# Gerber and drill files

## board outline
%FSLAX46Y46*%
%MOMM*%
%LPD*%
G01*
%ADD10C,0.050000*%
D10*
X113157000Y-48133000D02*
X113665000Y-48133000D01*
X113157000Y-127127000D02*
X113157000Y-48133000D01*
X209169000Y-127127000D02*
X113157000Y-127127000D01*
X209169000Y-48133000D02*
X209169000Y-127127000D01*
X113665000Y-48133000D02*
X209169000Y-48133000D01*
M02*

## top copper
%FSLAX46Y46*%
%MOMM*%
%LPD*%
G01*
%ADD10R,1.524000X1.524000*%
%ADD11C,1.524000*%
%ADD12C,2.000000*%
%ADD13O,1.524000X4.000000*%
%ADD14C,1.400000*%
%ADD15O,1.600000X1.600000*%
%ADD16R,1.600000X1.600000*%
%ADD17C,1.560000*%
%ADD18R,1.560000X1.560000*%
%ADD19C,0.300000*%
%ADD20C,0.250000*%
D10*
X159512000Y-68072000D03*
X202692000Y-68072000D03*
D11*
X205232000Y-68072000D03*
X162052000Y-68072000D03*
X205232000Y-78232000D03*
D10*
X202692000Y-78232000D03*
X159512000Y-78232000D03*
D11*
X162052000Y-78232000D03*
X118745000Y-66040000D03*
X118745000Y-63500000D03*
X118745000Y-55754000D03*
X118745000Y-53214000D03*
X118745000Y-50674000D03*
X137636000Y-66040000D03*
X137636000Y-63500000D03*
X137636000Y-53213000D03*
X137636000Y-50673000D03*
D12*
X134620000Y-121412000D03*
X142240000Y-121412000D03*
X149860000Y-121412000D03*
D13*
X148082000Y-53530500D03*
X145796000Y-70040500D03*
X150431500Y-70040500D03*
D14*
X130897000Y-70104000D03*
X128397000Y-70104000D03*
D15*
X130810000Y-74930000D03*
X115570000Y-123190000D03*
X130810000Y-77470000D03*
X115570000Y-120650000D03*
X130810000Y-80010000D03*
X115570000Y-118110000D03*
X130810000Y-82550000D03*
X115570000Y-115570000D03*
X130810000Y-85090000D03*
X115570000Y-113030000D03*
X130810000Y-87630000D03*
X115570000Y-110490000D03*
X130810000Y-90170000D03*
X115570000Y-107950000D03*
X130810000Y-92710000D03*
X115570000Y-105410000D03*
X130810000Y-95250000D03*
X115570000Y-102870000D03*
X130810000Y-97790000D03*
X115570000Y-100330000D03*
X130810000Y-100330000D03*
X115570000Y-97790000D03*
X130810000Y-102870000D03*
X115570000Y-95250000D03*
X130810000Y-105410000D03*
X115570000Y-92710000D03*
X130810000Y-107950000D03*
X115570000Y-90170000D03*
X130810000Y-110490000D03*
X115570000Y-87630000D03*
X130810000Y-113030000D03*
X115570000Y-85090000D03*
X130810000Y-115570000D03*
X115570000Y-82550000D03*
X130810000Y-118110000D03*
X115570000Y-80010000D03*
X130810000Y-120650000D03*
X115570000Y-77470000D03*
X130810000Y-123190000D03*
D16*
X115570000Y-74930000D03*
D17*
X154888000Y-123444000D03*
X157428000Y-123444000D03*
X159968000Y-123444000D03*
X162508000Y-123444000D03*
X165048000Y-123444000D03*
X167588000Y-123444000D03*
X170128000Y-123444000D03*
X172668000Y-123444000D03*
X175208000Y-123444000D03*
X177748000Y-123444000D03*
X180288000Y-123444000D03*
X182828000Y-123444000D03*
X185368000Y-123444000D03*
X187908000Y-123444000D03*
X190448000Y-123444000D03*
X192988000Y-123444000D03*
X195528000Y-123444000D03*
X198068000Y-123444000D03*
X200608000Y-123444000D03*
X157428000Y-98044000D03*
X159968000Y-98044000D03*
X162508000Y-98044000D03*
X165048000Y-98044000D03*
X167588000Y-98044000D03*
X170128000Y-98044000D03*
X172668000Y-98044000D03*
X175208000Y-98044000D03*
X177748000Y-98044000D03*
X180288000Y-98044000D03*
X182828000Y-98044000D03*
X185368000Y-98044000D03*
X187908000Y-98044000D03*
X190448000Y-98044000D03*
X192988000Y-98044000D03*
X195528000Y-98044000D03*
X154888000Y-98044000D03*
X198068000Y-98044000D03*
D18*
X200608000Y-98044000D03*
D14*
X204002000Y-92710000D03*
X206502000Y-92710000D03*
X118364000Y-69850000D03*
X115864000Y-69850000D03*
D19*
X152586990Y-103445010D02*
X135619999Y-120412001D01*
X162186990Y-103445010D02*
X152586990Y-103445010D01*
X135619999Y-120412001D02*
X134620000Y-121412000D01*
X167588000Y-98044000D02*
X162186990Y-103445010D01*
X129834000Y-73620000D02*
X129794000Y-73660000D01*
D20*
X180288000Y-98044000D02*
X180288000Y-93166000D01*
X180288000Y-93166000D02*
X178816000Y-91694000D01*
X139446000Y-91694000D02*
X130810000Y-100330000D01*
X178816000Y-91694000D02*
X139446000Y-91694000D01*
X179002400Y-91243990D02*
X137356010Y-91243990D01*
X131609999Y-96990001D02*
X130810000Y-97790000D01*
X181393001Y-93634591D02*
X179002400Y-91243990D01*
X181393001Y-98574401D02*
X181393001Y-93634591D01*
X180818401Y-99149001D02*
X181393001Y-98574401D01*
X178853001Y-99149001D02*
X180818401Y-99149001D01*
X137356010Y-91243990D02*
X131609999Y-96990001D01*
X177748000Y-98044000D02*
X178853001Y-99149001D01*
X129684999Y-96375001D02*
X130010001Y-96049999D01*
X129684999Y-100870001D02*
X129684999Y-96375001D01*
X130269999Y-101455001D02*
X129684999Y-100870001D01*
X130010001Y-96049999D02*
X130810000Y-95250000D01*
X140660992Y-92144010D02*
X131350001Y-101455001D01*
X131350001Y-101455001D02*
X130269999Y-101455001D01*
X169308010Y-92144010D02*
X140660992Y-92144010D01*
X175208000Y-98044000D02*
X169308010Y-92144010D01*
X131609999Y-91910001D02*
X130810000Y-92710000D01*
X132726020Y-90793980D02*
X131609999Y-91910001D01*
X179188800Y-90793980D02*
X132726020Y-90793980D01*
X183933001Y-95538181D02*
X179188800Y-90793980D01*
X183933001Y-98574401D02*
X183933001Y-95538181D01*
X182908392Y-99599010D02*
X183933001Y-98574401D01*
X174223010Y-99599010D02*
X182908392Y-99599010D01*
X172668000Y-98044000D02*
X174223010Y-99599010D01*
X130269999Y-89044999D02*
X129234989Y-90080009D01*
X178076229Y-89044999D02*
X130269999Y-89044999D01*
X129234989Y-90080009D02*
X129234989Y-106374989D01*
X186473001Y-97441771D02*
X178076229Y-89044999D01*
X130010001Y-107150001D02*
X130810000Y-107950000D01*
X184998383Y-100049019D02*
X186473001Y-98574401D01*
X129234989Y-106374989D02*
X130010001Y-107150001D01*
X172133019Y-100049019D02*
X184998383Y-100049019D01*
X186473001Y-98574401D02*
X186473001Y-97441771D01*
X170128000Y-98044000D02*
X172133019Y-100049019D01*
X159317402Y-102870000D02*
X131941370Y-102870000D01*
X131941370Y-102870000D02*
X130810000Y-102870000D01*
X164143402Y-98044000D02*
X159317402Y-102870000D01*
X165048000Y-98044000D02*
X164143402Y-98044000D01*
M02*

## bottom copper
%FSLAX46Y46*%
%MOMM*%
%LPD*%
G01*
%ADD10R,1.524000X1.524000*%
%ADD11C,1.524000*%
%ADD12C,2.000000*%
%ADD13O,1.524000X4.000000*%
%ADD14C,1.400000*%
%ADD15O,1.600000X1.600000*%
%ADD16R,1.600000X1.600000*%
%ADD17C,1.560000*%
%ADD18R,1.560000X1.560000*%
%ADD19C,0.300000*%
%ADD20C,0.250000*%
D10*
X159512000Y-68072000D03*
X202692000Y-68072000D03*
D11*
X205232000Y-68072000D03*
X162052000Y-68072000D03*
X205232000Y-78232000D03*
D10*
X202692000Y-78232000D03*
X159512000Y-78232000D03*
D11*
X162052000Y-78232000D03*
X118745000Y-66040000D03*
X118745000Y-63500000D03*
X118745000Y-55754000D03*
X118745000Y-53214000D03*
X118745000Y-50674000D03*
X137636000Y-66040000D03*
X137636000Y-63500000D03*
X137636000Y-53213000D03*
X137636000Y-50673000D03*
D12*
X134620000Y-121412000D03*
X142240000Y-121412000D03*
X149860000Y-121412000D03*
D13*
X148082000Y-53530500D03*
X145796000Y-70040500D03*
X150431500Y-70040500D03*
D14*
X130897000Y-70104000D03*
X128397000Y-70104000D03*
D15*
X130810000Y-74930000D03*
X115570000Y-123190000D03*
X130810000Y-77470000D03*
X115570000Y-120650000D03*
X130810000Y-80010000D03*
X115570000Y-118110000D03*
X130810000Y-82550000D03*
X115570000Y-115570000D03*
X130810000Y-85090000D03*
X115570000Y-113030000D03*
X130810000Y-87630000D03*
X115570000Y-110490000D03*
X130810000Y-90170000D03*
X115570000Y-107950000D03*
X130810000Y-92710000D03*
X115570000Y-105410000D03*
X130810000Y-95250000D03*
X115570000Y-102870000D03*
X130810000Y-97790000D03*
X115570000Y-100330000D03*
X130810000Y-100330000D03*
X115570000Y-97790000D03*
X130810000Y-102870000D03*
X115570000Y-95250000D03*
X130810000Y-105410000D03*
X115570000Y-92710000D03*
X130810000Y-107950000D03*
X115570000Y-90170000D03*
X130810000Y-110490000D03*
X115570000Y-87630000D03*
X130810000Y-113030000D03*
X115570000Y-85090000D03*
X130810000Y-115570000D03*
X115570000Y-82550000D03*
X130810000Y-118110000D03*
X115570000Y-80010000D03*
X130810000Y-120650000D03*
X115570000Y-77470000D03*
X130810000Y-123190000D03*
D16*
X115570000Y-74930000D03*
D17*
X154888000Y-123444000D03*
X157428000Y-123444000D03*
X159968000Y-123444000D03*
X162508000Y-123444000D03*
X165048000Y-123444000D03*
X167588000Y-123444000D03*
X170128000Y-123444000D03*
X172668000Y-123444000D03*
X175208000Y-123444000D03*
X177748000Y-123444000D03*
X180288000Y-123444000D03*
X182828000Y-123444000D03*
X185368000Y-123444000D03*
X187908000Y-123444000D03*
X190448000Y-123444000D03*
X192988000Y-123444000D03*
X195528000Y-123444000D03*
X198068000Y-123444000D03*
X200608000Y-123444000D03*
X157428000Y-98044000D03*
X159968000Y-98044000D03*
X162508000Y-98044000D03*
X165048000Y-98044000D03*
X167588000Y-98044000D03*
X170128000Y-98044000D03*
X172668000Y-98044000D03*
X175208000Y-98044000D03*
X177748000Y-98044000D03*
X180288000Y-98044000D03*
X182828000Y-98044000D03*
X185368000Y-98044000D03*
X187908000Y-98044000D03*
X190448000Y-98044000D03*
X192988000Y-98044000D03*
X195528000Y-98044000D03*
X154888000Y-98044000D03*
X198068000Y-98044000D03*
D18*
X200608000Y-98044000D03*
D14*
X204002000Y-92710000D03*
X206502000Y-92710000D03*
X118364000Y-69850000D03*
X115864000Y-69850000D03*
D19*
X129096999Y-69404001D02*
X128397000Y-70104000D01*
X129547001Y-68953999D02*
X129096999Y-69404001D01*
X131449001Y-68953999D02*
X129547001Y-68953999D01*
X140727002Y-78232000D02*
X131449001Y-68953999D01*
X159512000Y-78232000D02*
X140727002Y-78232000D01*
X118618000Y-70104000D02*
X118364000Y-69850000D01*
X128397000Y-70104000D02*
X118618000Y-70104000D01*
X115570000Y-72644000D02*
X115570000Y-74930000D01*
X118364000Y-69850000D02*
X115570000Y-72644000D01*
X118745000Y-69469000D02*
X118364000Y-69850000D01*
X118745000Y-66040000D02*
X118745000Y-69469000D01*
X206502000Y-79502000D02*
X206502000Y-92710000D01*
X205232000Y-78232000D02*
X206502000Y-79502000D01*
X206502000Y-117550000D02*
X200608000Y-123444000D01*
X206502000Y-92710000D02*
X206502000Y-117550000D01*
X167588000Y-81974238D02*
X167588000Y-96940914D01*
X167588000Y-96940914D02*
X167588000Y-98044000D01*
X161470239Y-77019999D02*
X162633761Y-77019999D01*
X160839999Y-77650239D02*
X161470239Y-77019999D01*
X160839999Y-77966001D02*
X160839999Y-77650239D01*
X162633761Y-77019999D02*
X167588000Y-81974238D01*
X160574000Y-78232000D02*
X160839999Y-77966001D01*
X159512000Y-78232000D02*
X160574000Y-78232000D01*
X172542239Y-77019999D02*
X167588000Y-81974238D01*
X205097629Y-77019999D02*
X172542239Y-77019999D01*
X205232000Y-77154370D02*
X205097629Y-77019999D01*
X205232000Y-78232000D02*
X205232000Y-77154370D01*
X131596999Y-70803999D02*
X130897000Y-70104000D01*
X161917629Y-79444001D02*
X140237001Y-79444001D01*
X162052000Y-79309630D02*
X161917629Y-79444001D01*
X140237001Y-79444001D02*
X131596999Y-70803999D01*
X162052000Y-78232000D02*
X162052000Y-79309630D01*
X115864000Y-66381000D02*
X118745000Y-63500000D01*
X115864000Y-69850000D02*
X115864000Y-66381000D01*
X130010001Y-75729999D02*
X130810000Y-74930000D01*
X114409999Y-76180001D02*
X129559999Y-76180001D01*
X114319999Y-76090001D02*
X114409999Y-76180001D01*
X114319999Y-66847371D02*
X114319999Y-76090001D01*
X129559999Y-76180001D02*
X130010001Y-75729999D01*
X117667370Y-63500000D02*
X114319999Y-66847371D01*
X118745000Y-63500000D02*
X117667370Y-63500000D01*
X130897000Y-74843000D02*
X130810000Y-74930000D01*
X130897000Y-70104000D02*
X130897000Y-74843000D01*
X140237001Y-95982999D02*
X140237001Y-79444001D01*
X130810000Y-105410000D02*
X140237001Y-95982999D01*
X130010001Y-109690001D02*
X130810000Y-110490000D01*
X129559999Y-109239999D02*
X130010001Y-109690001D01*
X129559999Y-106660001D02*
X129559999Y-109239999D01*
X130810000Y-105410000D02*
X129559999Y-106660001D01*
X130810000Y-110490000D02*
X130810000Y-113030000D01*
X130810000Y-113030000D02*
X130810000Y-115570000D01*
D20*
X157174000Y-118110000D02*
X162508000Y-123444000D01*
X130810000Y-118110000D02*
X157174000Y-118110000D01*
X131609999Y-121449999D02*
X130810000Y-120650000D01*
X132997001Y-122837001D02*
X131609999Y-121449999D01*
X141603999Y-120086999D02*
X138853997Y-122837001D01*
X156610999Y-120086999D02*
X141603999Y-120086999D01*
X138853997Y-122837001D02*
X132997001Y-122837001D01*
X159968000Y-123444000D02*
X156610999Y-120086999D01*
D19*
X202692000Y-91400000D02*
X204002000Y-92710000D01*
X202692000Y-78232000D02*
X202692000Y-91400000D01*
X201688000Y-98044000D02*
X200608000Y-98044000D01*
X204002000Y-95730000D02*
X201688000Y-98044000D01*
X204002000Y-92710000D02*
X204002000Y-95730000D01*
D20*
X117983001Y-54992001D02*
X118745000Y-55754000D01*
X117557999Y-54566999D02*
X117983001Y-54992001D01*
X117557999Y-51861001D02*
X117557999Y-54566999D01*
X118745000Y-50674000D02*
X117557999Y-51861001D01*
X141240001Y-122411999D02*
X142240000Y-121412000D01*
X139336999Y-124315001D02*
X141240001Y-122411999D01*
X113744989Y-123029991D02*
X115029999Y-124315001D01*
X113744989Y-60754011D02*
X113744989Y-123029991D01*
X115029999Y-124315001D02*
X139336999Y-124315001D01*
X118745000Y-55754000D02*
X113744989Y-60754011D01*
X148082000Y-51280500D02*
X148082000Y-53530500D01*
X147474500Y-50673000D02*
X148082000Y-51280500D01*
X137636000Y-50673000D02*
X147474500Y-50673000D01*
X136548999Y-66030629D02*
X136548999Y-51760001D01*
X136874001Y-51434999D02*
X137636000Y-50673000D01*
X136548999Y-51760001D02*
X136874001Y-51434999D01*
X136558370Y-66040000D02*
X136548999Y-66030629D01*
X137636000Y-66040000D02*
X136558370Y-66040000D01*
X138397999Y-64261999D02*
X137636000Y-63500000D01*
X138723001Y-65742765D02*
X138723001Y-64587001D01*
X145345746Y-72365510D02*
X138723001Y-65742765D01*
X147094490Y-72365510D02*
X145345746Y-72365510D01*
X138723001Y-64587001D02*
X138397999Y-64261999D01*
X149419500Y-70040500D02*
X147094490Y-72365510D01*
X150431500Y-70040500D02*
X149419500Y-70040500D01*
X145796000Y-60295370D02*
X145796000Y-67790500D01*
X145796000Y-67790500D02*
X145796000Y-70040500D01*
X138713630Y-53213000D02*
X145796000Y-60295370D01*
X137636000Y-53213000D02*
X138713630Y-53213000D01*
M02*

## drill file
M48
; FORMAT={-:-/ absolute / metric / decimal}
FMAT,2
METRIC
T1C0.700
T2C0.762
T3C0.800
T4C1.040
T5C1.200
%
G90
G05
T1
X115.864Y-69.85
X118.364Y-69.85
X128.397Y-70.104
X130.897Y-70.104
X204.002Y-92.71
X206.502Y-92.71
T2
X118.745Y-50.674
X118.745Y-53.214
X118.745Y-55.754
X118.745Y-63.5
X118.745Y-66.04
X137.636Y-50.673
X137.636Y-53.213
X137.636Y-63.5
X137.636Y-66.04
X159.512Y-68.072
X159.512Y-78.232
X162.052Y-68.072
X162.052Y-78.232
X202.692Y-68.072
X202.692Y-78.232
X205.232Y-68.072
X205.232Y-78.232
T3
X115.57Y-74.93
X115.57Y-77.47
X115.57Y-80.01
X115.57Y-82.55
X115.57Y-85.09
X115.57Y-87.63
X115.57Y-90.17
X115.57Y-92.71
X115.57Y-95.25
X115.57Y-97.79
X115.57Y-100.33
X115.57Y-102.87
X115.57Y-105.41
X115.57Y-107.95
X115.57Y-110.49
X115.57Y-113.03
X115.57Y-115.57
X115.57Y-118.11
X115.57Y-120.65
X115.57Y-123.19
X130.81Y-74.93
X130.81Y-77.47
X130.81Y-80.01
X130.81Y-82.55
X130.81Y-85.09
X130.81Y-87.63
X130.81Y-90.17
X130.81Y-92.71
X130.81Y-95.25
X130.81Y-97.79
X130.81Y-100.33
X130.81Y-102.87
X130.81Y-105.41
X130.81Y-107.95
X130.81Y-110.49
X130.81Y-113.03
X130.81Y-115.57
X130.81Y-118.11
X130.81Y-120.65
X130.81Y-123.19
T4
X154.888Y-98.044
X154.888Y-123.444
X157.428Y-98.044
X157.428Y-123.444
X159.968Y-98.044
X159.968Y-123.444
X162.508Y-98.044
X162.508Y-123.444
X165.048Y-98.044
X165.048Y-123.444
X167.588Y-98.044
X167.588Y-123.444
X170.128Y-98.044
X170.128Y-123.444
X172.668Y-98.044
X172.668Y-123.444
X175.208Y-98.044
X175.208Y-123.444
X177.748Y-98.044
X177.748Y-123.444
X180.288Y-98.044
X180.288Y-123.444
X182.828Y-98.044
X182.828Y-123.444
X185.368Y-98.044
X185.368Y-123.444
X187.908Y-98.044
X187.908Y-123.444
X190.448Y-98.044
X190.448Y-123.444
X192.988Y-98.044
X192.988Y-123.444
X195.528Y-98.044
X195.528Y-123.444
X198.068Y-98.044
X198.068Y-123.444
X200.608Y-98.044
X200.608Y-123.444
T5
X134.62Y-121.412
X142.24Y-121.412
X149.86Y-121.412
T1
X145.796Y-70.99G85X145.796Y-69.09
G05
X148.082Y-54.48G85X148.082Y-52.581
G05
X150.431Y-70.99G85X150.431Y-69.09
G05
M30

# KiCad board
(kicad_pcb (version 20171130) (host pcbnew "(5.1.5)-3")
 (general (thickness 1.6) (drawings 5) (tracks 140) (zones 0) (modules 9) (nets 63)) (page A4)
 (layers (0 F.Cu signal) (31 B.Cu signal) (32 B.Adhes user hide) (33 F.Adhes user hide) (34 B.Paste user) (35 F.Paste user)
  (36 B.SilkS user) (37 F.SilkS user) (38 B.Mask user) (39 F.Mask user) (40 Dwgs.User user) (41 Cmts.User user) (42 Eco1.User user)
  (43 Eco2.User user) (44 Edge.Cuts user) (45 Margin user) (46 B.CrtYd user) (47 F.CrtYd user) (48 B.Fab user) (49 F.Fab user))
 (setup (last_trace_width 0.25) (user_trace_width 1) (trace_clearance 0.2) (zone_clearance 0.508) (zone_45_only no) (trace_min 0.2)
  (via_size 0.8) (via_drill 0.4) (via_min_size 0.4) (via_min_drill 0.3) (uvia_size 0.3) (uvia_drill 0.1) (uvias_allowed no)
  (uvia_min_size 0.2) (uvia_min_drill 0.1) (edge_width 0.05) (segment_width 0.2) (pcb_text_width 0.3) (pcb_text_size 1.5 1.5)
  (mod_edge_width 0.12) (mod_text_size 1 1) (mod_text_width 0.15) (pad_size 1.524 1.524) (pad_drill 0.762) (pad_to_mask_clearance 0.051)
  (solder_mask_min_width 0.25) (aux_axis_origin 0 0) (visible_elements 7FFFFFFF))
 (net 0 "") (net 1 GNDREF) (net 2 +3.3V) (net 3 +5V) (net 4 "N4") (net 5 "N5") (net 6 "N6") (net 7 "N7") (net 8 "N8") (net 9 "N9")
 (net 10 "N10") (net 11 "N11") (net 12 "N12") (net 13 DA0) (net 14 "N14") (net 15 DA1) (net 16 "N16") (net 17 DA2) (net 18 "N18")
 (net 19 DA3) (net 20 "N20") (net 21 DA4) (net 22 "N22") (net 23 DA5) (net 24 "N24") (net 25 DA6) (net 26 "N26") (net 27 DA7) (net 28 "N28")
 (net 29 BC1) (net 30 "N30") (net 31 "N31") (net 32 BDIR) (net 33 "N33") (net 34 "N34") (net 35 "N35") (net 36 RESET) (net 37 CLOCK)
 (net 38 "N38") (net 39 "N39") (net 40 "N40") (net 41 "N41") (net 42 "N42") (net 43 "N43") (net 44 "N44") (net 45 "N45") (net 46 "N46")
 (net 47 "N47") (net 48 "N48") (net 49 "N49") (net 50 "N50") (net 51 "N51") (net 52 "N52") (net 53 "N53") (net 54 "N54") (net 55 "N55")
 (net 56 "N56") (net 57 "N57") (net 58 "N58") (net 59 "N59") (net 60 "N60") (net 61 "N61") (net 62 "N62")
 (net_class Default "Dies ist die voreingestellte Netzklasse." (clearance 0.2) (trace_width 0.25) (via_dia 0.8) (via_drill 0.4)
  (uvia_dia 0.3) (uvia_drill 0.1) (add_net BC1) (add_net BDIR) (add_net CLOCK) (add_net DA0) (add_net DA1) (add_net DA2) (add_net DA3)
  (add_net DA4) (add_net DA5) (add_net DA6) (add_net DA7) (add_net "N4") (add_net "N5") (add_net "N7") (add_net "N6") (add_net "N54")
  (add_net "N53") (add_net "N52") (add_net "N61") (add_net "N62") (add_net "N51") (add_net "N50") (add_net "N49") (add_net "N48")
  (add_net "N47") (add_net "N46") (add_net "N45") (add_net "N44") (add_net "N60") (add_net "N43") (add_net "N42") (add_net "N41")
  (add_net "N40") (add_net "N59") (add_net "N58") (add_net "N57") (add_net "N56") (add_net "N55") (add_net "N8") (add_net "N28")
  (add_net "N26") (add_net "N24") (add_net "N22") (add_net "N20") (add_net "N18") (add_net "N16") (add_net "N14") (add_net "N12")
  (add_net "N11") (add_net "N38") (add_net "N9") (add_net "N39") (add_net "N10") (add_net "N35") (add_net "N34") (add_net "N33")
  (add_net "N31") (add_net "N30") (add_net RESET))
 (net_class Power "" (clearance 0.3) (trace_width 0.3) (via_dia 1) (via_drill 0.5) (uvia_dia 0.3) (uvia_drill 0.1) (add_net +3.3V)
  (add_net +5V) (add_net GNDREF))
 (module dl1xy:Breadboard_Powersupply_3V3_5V (layer F.Cu) (at 182.372 60.198)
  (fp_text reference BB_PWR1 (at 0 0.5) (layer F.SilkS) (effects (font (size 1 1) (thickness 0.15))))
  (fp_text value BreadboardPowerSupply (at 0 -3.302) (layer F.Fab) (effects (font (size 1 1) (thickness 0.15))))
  (pad 5 thru_hole rect (at -22.86 7.874) (size 1.524 1.524) (drill 0.762) (layers *.Cu *.Mask))
  (pad 7 thru_hole rect (at 20.32 7.874) (size 1.524 1.524) (drill 0.762) (layers *.Cu *.Mask))
  (pad 8 thru_hole circle (at 22.86 7.874) (size 1.524 1.524) (drill 0.762) (layers *.Cu *.Mask))
  (pad 6 thru_hole circle (at -20.32 7.874) (size 1.524 1.524) (drill 0.762) (layers *.Cu *.Mask))
  (pad 4 thru_hole circle (at 22.86 18.034) (size 1.524 1.524) (drill 0.762) (layers *.Cu *.Mask) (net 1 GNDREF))
  (pad 3 thru_hole rect (at 20.32 18.034) (size 1.524 1.524) (drill 0.762) (layers *.Cu *.Mask) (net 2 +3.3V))
  (pad 2 thru_hole rect (at -22.86 18.034) (size 1.524 1.524) (drill 0.762) (layers *.Cu *.Mask) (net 1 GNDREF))
  (pad 1 thru_hole circle (at -20.32 18.034) (size 1.524 1.524) (drill 0.762) (layers *.Cu *.Mask) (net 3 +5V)))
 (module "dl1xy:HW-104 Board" (layer F.Cu) (at 140.716 58.42 270)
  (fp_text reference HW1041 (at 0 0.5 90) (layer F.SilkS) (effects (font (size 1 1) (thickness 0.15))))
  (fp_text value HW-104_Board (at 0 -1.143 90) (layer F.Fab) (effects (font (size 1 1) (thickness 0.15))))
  (pad 5 thru_hole circle (at 7.62 21.971 270) (size 1.524 1.524) (drill 0.762) (layers *.Cu *.Mask) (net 1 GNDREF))
  (pad 4 thru_hole circle (at 5.08 21.971 270) (size 1.524 1.524) (drill 0.762) (layers *.Cu *.Mask) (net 3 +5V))
  (pad 3 thru_hole circle (at -2.666 21.971 270) (size 1.524 1.524) (drill 0.762) (layers *.Cu *.Mask) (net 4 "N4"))
  (pad 2 thru_hole circle (at -5.206 21.971 270) (size 1.524 1.524) (drill 0.762) (layers *.Cu *.Mask) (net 1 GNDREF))
  (pad 1 thru_hole circle (at -7.746 21.971 270) (size 1.524 1.524) (drill 0.762) (layers *.Cu *.Mask) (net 4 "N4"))
  (pad 9 thru_hole circle (at 7.62 3.08 270) (size 1.524 1.524) (drill 0.762) (layers *.Cu *.Mask) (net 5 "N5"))
  (pad 8 thru_hole circle (at 5.08 3.08 270) (size 1.524 1.524) (drill 0.762) (layers *.Cu *.Mask) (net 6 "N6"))
  (pad 7 thru_hole circle (at -5.207 3.08 270) (size 1.524 1.524) (drill 0.762) (layers *.Cu *.Mask) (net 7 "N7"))
  (pad 6 thru_hole circle (at -7.747 3.08 270) (size 1.524 1.524) (drill 0.762) (layers *.Cu *.Mask) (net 5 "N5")))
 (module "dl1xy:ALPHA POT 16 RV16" (layer F.Cu) (at 142.24 116.459)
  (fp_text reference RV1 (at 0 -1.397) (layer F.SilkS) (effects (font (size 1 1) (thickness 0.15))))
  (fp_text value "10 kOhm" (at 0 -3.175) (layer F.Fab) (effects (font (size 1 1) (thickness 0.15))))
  (pad 1 thru_hole circle (at -7.62 4.953) (size 2 2) (drill 1.2) (layers *.Cu *.Mask) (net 1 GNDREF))
  (pad 2 thru_hole circle (at 0 4.953) (size 2 2) (drill 1.2) (layers *.Cu *.Mask) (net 4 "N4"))
  (pad 3 thru_hole circle (at 7.62 4.953) (size 2 2) (drill 1.2) (layers *.Cu *.Mask) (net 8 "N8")))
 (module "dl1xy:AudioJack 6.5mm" (layer F.Cu) (at 148.082 76.708 180)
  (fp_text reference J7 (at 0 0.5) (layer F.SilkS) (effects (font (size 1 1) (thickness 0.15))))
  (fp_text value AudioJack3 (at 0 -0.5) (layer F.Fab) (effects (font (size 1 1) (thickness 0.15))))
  (pad S thru_hole oval (at 0 23.1775 180) (size 1.524 4) (drill oval 0.7 2.6) (layers *.Cu *.Mask) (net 5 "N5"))
  (pad T thru_hole oval (at 2.286 6.6675 180) (size 1.524 4) (drill oval 0.7 2.6) (layers *.Cu *.Mask) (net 7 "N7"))
  (pad R thru_hole oval (at -2.3495 6.6675 180) (size 1.524 4) (drill oval 0.7 2.6) (layers *.Cu *.Mask) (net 6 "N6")))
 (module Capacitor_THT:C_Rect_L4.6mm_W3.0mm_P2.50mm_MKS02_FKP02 (layer F.Cu) (at 128.397 70.104)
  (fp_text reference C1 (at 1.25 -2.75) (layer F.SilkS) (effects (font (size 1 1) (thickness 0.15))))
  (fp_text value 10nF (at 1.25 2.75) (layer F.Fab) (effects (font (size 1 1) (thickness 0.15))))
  (pad 2 thru_hole circle (at 2.5 0) (size 1.4 1.4) (drill 0.7) (layers *.Cu *.Mask) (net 3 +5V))
  (pad 1 thru_hole circle (at 0 0) (size 1.4 1.4) (drill 0.7) (layers *.Cu *.Mask) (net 1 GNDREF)))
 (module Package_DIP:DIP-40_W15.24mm (layer F.Cu) (at 115.57 74.93)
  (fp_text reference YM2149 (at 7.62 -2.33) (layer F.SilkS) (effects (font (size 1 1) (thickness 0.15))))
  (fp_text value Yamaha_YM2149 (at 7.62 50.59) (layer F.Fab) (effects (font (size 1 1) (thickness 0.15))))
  (pad 40 thru_hole oval (at 15.24 0) (size 1.6 1.6) (drill 0.8) (layers *.Cu *.Mask) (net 3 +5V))
  (pad 20 thru_hole oval (at 0 48.26) (size 1.6 1.6) (drill 0.8) (layers *.Cu *.Mask) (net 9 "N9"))
  (pad 39 thru_hole oval (at 15.24 2.54) (size 1.6 1.6) (drill 0.8) (layers *.Cu *.Mask) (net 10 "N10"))
  (pad 19 thru_hole oval (at 0 45.72) (size 1.6 1.6) (drill 0.8) (layers *.Cu *.Mask) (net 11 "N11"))
  (pad 38 thru_hole oval (at 15.24 5.08) (size 1.6 1.6) (drill 0.8) (layers *.Cu *.Mask) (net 8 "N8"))
  (pad 18 thru_hole oval (at 0 43.18) (size 1.6 1.6) (drill 0.8) (layers *.Cu *.Mask) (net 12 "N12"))
  (pad 37 thru_hole oval (at 15.24 7.62) (size 1.6 1.6) (drill 0.8) (layers *.Cu *.Mask) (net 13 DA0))
  (pad 17 thru_hole oval (at 0 40.64) (size 1.6 1.6) (drill 0.8) (layers *.Cu *.Mask) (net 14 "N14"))
  (pad 36 thru_hole oval (at 15.24 10.16) (size 1.6 1.6) (drill 0.8) (layers *.Cu *.Mask) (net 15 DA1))
  (pad 16 thru_hole oval (at 0 38.1) (size 1.6 1.6) (drill 0.8) (layers *.Cu *.Mask) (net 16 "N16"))
  (pad 35 thru_hole oval (at 15.24 12.7) (size 1.6 1.6) (drill 0.8) (layers *.Cu *.Mask) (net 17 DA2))
  (pad 15 thru_hole oval (at 0 35.56) (size 1.6 1.6) (drill 0.8) (layers *.Cu *.Mask) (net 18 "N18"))
  (pad 34 thru_hole oval (at 15.24 15.24) (size 1.6 1.6) (drill 0.8) (layers *.Cu *.Mask) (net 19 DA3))
  (pad 14 thru_hole oval (at 0 33.02) (size 1.6 1.6) (drill 0.8) (layers *.Cu *.Mask) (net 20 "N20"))
  (pad 33 thru_hole oval (at 15.24 17.78) (size 1.6 1.6) (drill 0.8) (layers *.Cu *.Mask) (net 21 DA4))
  (pad 13 thru_hole oval (at 0 30.48) (size 1.6 1.6) (drill 0.8) (layers *.Cu *.Mask) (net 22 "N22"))
  (pad 32 thru_hole oval (at 15.24 20.32) (size 1.6 1.6) (drill 0.8) (layers *.Cu *.Mask) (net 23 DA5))
  (pad 12 thru_hole oval (at 0 27.94) (size 1.6 1.6) (drill 0.8) (layers *.Cu *.Mask) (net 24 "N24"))
  (pad 31 thru_hole oval (at 15.24 22.86) (size 1.6 1.6) (drill 0.8) (layers *.Cu *.Mask) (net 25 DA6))
  (pad 11 thru_hole oval (at 0 25.4) (size 1.6 1.6) (drill 0.8) (layers *.Cu *.Mask) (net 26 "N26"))
  (pad 30 thru_hole oval (at 15.24 25.4) (size 1.6 1.6) (drill 0.8) (layers *.Cu *.Mask) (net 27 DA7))
  (pad 10 thru_hole oval (at 0 22.86) (size 1.6 1.6) (drill 0.8) (layers *.Cu *.Mask) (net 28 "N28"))
  (pad 29 thru_hole oval (at 15.24 27.94) (size 1.6 1.6) (drill 0.8) (layers *.Cu *.Mask) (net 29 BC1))
  (pad 9 thru_hole oval (at 0 20.32) (size 1.6 1.6) (drill 0.8) (layers *.Cu *.Mask) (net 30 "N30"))
  (pad 28 thru_hole oval (at 15.24 30.48) (size 1.6 1.6) (drill 0.8) (layers *.Cu *.Mask) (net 3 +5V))
  (pad 8 thru_hole oval (at 0 17.78) (size 1.6 1.6) (drill 0.8) (layers *.Cu *.Mask) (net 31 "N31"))
  (pad 27 thru_hole oval (at 15.24 33.02) (size 1.6 1.6) (drill 0.8) (layers *.Cu *.Mask) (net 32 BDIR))
  (pad 7 thru_hole oval (at 0 15.24) (size 1.6 1.6) (drill 0.8) (layers *.Cu *.Mask) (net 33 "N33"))
  (pad 26 thru_hole oval (at 15.24 35.56) (size 1.6 1.6) (drill 0.8) (layers *.Cu *.Mask) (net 3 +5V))
  (pad 6 thru_hole oval (at 0 12.7) (size 1.6 1.6) (drill 0.8) (layers *.Cu *.Mask) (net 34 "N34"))
  (pad 25 thru_hole oval (at 15.24 38.1) (size 1.6 1.6) (drill 0.8) (layers *.Cu *.Mask) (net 3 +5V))
  (pad 5 thru_hole oval (at 0 10.16) (size 1.6 1.6) (drill 0.8) (layers *.Cu *.Mask) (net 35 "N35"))
  (pad 24 thru_hole oval (at 15.24 40.64) (size 1.6 1.6) (drill 0.8) (layers *.Cu *.Mask) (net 3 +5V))
  (pad 4 thru_hole oval (at 0 7.62) (size 1.6 1.6) (drill 0.8) (layers *.Cu *.Mask) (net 8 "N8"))
  (pad 23 thru_hole oval (at 15.24 43.18) (size 1.6 1.6) (drill 0.8) (layers *.Cu *.Mask) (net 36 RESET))
  (pad 3 thru_hole oval (at 0 5.08) (size 1.6 1.6) (drill 0.8) (layers *.Cu *.Mask) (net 8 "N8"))
  (pad 22 thru_hole oval (at 15.24 45.72) (size 1.6 1.6) (drill 0.8) (layers *.Cu *.Mask) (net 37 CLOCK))
  (pad 2 thru_hole oval (at 0 2.54) (size 1.6 1.6) (drill 0.8) (layers *.Cu *.Mask) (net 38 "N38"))
  (pad 21 thru_hole oval (at 15.24 48.26) (size 1.6 1.6) (drill 0.8) (layers *.Cu *.Mask) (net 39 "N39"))
  (pad 1 thru_hole rect (at 0 0) (size 1.6 1.6) (drill 0.8) (layers *.Cu *.Mask) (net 1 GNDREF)))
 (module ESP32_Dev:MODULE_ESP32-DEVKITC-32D (layer F.Cu) (at 180.848 110.744 270)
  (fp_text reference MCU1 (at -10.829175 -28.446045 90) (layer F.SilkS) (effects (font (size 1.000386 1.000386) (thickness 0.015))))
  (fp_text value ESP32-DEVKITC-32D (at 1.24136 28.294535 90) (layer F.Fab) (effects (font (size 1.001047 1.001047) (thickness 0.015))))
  (pad 38 thru_hole circle (at 12.7 25.96 270) (size 1.56 1.56) (drill 1.04) (layers *.Cu *.Mask) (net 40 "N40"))
  (pad 37 thru_hole circle (at 12.7 23.42 270) (size 1.56 1.56) (drill 1.04) (layers *.Cu *.Mask) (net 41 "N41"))
  (pad 36 thru_hole circle (at 12.7 20.88 270) (size 1.56 1.56) (drill 1.04) (layers *.Cu *.Mask) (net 37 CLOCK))
  (pad 35 thru_hole circle (at 12.7 18.34 270) (size 1.56 1.56) (drill 1.04) (layers *.Cu *.Mask) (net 36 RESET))
  (pad 34 thru_hole circle (at 12.7 15.8 270) (size 1.56 1.56) (drill 1.04) (layers *.Cu *.Mask) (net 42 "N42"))
  (pad 33 thru_hole circle (at 12.7 13.26 270) (size 1.56 1.56) (drill 1.04) (layers *.Cu *.Mask) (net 13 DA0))
  (pad 32 thru_hole circle (at 12.7 10.72 270) (size 1.56 1.56) (drill 1.04) (layers *.Cu *.Mask) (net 15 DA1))
  (pad 31 thru_hole circle (at 12.7 8.18 270) (size 1.56 1.56) (drill 1.04) (layers *.Cu *.Mask) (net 17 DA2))
  (pad 30 thru_hole circle (at 12.7 5.64 270) (size 1.56 1.56) (drill 1.04) (layers *.Cu *.Mask) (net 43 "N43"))
  (pad 29 thru_hole circle (at 12.7 3.1 270) (size 1.56 1.56) (drill 1.04) (layers *.Cu *.Mask) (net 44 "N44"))
  (pad 28 thru_hole circle (at 12.7 0.56 270) (size 1.56 1.56) (drill 1.04) (layers *.Cu *.Mask) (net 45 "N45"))
  (pad 27 thru_hole circle (at 12.7 -1.98 270) (size 1.56 1.56) (drill 1.04) (layers *.Cu *.Mask) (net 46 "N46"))
  (pad 26 thru_hole circle (at 12.7 -4.52 270) (size 1.56 1.56) (drill 1.04) (layers *.Cu *.Mask) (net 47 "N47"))
  (pad 25 thru_hole circle (at 12.7 -7.06 270) (size 1.56 1.56) (drill 1.04) (layers *.Cu *.Mask) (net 19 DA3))
  (pad 24 thru_hole circle (at 12.7 -9.6 270) (size 1.56 1.56) (drill 1.04) (layers *.Cu *.Mask) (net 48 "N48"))
  (pad 23 thru_hole circle (at 12.7 -12.14 270) (size 1.56 1.56) (drill 1.04) (layers *.Cu *.Mask) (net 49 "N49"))
  (pad 22 thru_hole circle (at 12.7 -14.68 270) (size 1.56 1.56) (drill 1.04) (layers *.Cu *.Mask) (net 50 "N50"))
  (pad 21 thru_hole circle (at 12.7 -17.22 270) (size 1.56 1.56) (drill 1.04) (layers *.Cu *.Mask) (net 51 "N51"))
  (pad 20 thru_hole circle (at 12.7 -19.76 270) (size 1.56 1.56) (drill 1.04) (layers *.Cu *.Mask) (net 1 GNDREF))
  (pad 18 thru_hole circle (at -12.7 23.42 270) (size 1.56 1.56) (drill 1.04) (layers *.Cu *.Mask) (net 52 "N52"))
  (pad 17 thru_hole circle (at -12.7 20.88 270) (size 1.56 1.56) (drill 1.04) (layers *.Cu *.Mask) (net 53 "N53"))
  (pad 16 thru_hole circle (at -12.7 18.34 270) (size 1.56 1.56) (drill 1.04) (layers *.Cu *.Mask) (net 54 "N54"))
  (pad 15 thru_hole circle (at -12.7 15.8 270) (size 1.56 1.56) (drill 1.04) (layers *.Cu *.Mask) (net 29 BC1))
  (pad 14 thru_hole circle (at -12.7 13.26 270) (size 1.56 1.56) (drill 1.04) (layers *.Cu *.Mask) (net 1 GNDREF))
  (pad 13 thru_hole circle (at -12.7 10.72 270) (size 1.56 1.56) (drill 1.04) (layers *.Cu *.Mask) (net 32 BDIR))
  (pad 12 thru_hole circle (at -12.7 8.18 270) (size 1.56 1.56) (drill 1.04) (layers *.Cu *.Mask) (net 21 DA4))
  (pad 11 thru_hole circle (at -12.7 5.64 270) (size 1.56 1.56) (drill 1.04) (layers *.Cu *.Mask) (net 23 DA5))
  (pad 10 thru_hole circle (at -12.7 3.1 270) (size 1.56 1.56) (drill 1.04) (layers *.Cu *.Mask) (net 25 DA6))
  (pad 9 thru_hole circle (at -12.7 0.56 270) (size 1.56 1.56) (drill 1.04) (layers *.Cu *.Mask) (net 27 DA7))
  (pad 8 thru_hole circle (at -12.7 -1.98 270) (size 1.56 1.56) (drill 1.04) (layers *.Cu *.Mask) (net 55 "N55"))
  (pad 7 thru_hole circle (at -12.7 -4.52 270) (size 1.56 1.56) (drill 1.04) (layers *.Cu *.Mask) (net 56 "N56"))
  (pad 6 thru_hole circle (at -12.7 -7.06 270) (size 1.56 1.56) (drill 1.04) (layers *.Cu *.Mask) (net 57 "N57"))
  (pad 5 thru_hole circle (at -12.7 -9.6 270) (size 1.56 1.56) (drill 1.04) (layers *.Cu *.Mask) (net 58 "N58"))
  (pad 4 thru_hole circle (at -12.7 -12.14 270) (size 1.56 1.56) (drill 1.04) (layers *.Cu *.Mask) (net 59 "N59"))
  (pad 3 thru_hole circle (at -12.7 -14.68 270) (size 1.56 1.56) (drill 1.04) (layers *.Cu *.Mask) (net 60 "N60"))
  (pad 19 thru_hole circle (at -12.7 25.96 270) (size 1.56 1.56) (drill 1.04) (layers *.Cu *.Mask) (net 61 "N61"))
  (pad 2 thru_hole circle (at -12.7 -17.22 270) (size 1.56 1.56) (drill 1.04) (layers *.Cu *.Mask) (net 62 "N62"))
  (pad 1 thru_hole rect (at -12.7 -19.76 270) (size 1.56 1.56) (drill 1.04) (layers *.Cu *.Mask) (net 2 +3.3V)))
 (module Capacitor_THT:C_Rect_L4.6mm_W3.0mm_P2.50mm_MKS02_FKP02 (layer F.Cu) (at 206.502 92.71 180)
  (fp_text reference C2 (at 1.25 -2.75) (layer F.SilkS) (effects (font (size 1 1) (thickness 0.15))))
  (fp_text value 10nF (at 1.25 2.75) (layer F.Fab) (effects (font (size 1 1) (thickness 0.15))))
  (pad 2 thru_hole circle (at 2.5 0 180) (size 1.4 1.4) (drill 0.7) (layers *.Cu *.Mask) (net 2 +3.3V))
  (pad 1 thru_hole circle (at 0 0 180) (size 1.4 1.4) (drill 0.7) (layers *.Cu *.Mask) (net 1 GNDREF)))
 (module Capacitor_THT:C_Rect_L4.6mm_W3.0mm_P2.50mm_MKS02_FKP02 (layer F.Cu) (at 118.364 69.85 180)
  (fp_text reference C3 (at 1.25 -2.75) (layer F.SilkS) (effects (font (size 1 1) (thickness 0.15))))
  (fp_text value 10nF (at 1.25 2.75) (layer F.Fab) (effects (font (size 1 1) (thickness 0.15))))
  (pad 1 thru_hole circle (at 0 0 180) (size 1.4 1.4) (drill 0.7) (layers *.Cu *.Mask) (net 1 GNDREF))
  (pad 2 thru_hole circle (at 2.5 0 180) (size 1.4 1.4) (drill 0.7) (layers *.Cu *.Mask) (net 3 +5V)))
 (gr_line (start 113.157 48.133) (end 113.665 48.133) (layer Edge.Cuts) (width 0.05))
 (gr_line (start 113.157 127.127) (end 113.157 48.133) (layer Edge.Cuts) (width 0.05))
 (gr_line (start 209.169 127.127) (end 113.157 127.127) (layer Edge.Cuts) (width 0.05))
 (gr_line (start 209.169 48.133) (end 209.169 127.127) (layer Edge.Cuts) (width 0.05))
 (gr_line (start 113.665 48.133) (end 209.169 48.133) (layer Edge.Cuts) (width 0.05))
 (segment (start 129.096999 69.404001) (end 128.397 70.104) (width 0.3) (layer B.Cu) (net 1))
 (segment (start 129.547001 68.953999) (end 129.096999 69.404001) (width 0.3) (layer B.Cu) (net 1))
 (segment (start 131.449001 68.953999) (end 129.547001 68.953999) (width 0.3) (layer B.Cu) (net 1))
 (segment (start 140.727002 78.232) (end 131.449001 68.953999) (width 0.3) (layer B.Cu) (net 1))
 (segment (start 159.512 78.232) (end 140.727002 78.232) (width 0.3) (layer B.Cu) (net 1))
 (segment (start 118.618 70.104) (end 118.364 69.85) (width 0.3) (layer B.Cu) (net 1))
 (segment (start 128.397 70.104) (end 118.618 70.104) (width 0.3) (layer B.Cu) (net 1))
 (segment (start 115.57 72.644) (end 115.57 74.93) (width 0.3) (layer B.Cu) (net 1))
 (segment (start 118.364 69.85) (end 115.57 72.644) (width 0.3) (layer B.Cu) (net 1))
 (segment (start 118.745 69.469) (end 118.364 69.85) (width 0.3) (layer B.Cu) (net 1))
 (segment (start 118.745 66.04) (end 118.745 69.469) (width 0.3) (layer B.Cu) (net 1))
 (segment (start 206.502 79.502) (end 206.502 92.71) (width 0.3) (layer B.Cu) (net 1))
 (segment (start 205.232 78.232) (end 206.502 79.502) (width 0.3) (layer B.Cu) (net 1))
 (segment (start 206.502 117.55) (end 200.608 123.444) (width 0.3) (layer B.Cu) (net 1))
 (segment (start 206.502 92.71) (end 206.502 117.55) (width 0.3) (layer B.Cu) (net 1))
 (segment (start 167.588 81.974238) (end 167.588 96.940914) (width 0.3) (layer B.Cu) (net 1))
 (segment (start 167.588 96.940914) (end 167.588 98.044) (width 0.3) (layer B.Cu) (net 1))
 (segment (start 161.470239 77.019999) (end 162.633761 77.019999) (width 0.3) (layer B.Cu) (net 1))
 (segment (start 160.839999 77.650239) (end 161.470239 77.019999) (width 0.3) (layer B.Cu) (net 1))
 (segment (start 160.839999 77.966001) (end 160.839999 77.650239) (width 0.3) (layer B.Cu) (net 1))
 (segment (start 162.633761 77.019999) (end 167.588 81.974238) (width 0.3) (layer B.Cu) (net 1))
 (segment (start 160.574 78.232) (end 160.839999 77.966001) (width 0.3) (layer B.Cu) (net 1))
 (segment (start 159.512 78.232) (end 160.574 78.232) (width 0.3) (layer B.Cu) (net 1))
 (segment (start 172.542239 77.019999) (end 167.588 81.974238) (width 0.3) (layer B.Cu) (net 1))
 (segment (start 205.097629 77.019999) (end 172.542239 77.019999) (width 0.3) (layer B.Cu) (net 1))
 (segment (start 205.232 77.15437) (end 205.097629 77.019999) (width 0.3) (layer B.Cu) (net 1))
 (segment (start 205.232 78.232) (end 205.232 77.15437) (width 0.3) (layer B.Cu) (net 1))
 (segment (start 152.58699 103.44501) (end 135.619999 120.412001) (width 0.3) (layer F.Cu) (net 1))
 (segment (start 162.18699 103.44501) (end 152.58699 103.44501) (width 0.3) (layer F.Cu) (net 1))
 (segment (start 135.619999 120.412001) (end 134.62 121.412) (width 0.3) (layer F.Cu) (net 1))
 (segment (start 167.588 98.044) (end 162.18699 103.44501) (width 0.3) (layer F.Cu) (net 1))
 (segment (start 129.834 73.62) (end 129.794 73.66) (width 0.3) (layer F.Cu) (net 3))
 (segment (start 131.596999 70.803999) (end 130.897 70.104) (width 0.3) (layer B.Cu) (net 3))
 (segment (start 161.917629 79.444001) (end 140.237001 79.444001) (width 0.3) (layer B.Cu) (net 3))
 (segment (start 162.052 79.30963) (end 161.917629 79.444001) (width 0.3) (layer B.Cu) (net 3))
 (segment (start 140.237001 79.444001) (end 131.596999 70.803999) (width 0.3) (layer B.Cu) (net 3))
 (segment (start 162.052 78.232) (end 162.052 79.30963) (width 0.3) (layer B.Cu) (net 3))
 (segment (start 115.864 66.381) (end 118.745 63.5) (width 0.3) (layer B.Cu) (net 3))
 (segment (start 115.864 69.85) (end 115.864 66.381) (width 0.3) (layer B.Cu) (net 3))
 (segment (start 130.010001 75.729999) (end 130.81 74.93) (width 0.3) (layer B.Cu) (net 3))
 (segment (start 114.409999 76.180001) (end 129.559999 76.180001) (width 0.3) (layer B.Cu) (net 3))
 (segment (start 114.319999 76.090001) (end 114.409999 76.180001) (width 0.3) (layer B.Cu) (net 3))
 (segment (start 114.319999 66.847371) (end 114.319999 76.090001) (width 0.3) (layer B.Cu) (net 3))
 (segment (start 129.559999 76.180001) (end 130.010001 75.729999) (width 0.3) (layer B.Cu) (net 3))
 (segment (start 117.66737 63.5) (end 114.319999 66.847371) (width 0.3) (layer B.Cu) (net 3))
 (segment (start 118.745 63.5) (end 117.66737 63.5) (width 0.3) (layer B.Cu) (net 3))
 (segment (start 130.897 74.843) (end 130.81 74.93) (width 0.3) (layer B.Cu) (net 3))
 (segment (start 130.897 70.104) (end 130.897 74.843) (width 0.3) (layer B.Cu) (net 3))
 (segment (start 140.237001 95.982999) (end 140.237001 79.444001) (width 0.3) (layer B.Cu) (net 3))
 (segment (start 130.81 105.41) (end 140.237001 95.982999) (width 0.3) (layer B.Cu) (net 3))
 (segment (start 130.010001 109.690001) (end 130.81 110.49) (width 0.3) (layer B.Cu) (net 3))
 (segment (start 129.559999 109.239999) (end 130.010001 109.690001) (width 0.3) (layer B.Cu) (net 3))
 (segment (start 129.559999 106.660001) (end 129.559999 109.239999) (width 0.3) (layer B.Cu) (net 3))
 (segment (start 130.81 105.41) (end 129.559999 106.660001) (width 0.3) (layer B.Cu) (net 3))
 (segment (start 130.81 110.49) (end 130.81 113.03) (width 0.3) (layer B.Cu) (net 3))
 (segment (start 130.81 113.03) (end 130.81 115.57) (width 0.3) (layer B.Cu) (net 3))
 (segment (start 180.288 98.044) (end 180.288 93.166) (width 0.25) (layer F.Cu) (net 27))
 (segment (start 180.288 93.166) (end 178.816 91.694) (width 0.25) (layer F.Cu) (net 27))
 (segment (start 139.446 91.694) (end 130.81 100.33) (width 0.25) (layer F.Cu) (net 27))
 (segment (start 178.816 91.694) (end 139.446 91.694) (width 0.25) (layer F.Cu) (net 27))
 (segment (start 179.0024 91.24399) (end 137.35601 91.24399) (width 0.25) (layer F.Cu) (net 25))
 (segment (start 131.609999 96.990001) (end 130.81 97.79) (width 0.25) (layer F.Cu) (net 25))
 (segment (start 181.393001 93.634591) (end 179.0024 91.24399) (width 0.25) (layer F.Cu) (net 25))
 (segment (start 181.393001 98.574401) (end 181.393001 93.634591) (width 0.25) (layer F.Cu) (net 25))
 (segment (start 180.818401 99.149001) (end 181.393001 98.574401) (width 0.25) (layer F.Cu) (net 25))
 (segment (start 178.853001 99.149001) (end 180.818401 99.149001) (width 0.25) (layer F.Cu) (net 25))
 (segment (start 137.35601 91.24399) (end 131.609999 96.990001) (width 0.25) (layer F.Cu) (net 25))
 (segment (start 177.748 98.044) (end 178.853001 99.149001) (width 0.25) (layer F.Cu) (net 25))
 (segment (start 129.684999 96.375001) (end 130.010001 96.049999) (width 0.25) (layer F.Cu) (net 23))
 (segment (start 129.684999 100.870001) (end 129.684999 96.375001) (width 0.25) (layer F.Cu) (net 23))
 (segment (start 130.269999 101.455001) (end 129.684999 100.870001) (width 0.25) (layer F.Cu) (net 23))
 (segment (start 130.010001 96.049999) (end 130.81 95.25) (width 0.25) (layer F.Cu) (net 23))
 (segment (start 140.660992 92.14401) (end 131.350001 101.455001) (width 0.25) (layer F.Cu) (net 23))
 (segment (start 131.350001 101.455001) (end 130.269999 101.455001) (width 0.25) (layer F.Cu) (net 23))
 (segment (start 169.30801 92.14401) (end 140.660992 92.14401) (width 0.25) (layer F.Cu) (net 23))
 (segment (start 175.208 98.044) (end 169.30801 92.14401) (width 0.25) (layer F.Cu) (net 23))
 (segment (start 131.609999 91.910001) (end 130.81 92.71) (width 0.25) (layer F.Cu) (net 21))
 (segment (start 132.72602 90.79398) (end 131.609999 91.910001) (width 0.25) (layer F.Cu) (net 21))
 (segment (start 179.1888 90.79398) (end 132.72602 90.79398) (width 0.25) (layer F.Cu) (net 21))
 (segment (start 183.933001 95.538181) (end 179.1888 90.79398) (width 0.25) (layer F.Cu) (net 21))
 (segment (start 183.933001 98.574401) (end 183.933001 95.538181) (width 0.25) (layer F.Cu) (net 21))
 (segment (start 182.908392 99.59901) (end 183.933001 98.574401) (width 0.25) (layer F.Cu) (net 21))
 (segment (start 174.22301 99.59901) (end 182.908392 99.59901) (width 0.25) (layer F.Cu) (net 21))
 (segment (start 172.668 98.044) (end 174.22301 99.59901) (width 0.25) (layer F.Cu) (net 21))
 (segment (start 130.269999 89.044999) (end 129.234989 90.080009) (width 0.25) (layer F.Cu) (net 32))
 (segment (start 178.076229 89.044999) (end 130.269999 89.044999) (width 0.25) (layer F.Cu) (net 32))
 (segment (start 129.234989 90.080009) (end 129.234989 106.374989) (width 0.25) (layer F.Cu) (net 32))
 (segment (start 186.473001 97.441771) (end 178.076229 89.044999) (width 0.25) (layer F.Cu) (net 32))
 (segment (start 130.010001 107.150001) (end 130.81 107.95) (width 0.25) (layer F.Cu) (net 32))
 (segment (start 184.998383 100.049019) (end 186.473001 98.574401) (width 0.25) (layer F.Cu) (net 32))
 (segment (start 129.234989 106.374989) (end 130.010001 107.150001) (width 0.25) (layer F.Cu) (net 32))
 (segment (start 172.133019 100.049019) (end 184.998383 100.049019) (width 0.25) (layer F.Cu) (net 32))
 (segment (start 186.473001 98.574401) (end 186.473001 97.441771) (width 0.25) (layer F.Cu) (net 32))
 (segment (start 170.128 98.044) (end 172.133019 100.049019) (width 0.25) (layer F.Cu) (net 32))
 (segment (start 159.317402 102.87) (end 131.94137 102.87) (width 0.25) (layer F.Cu) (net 29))
 (segment (start 131.94137 102.87) (end 130.81 102.87) (width 0.25) (layer F.Cu) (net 29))
 (segment (start 164.143402 98.044) (end 159.317402 102.87) (width 0.25) (layer F.Cu) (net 29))
 (segment (start 165.048 98.044) (end 164.143402 98.044) (width 0.25) (layer F.Cu) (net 29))
 (segment (start 157.174 118.11) (end 162.508 123.444) (width 0.25) (layer B.Cu) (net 36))
 (segment (start 130.81 118.11) (end 157.174 118.11) (width 0.25) (layer B.Cu) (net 36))
 (segment (start 131.609999 121.449999) (end 130.81 120.65) (width 0.25) (layer B.Cu) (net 37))
 (segment (start 132.997001 122.837001) (end 131.609999 121.449999) (width 0.25) (layer B.Cu) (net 37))
 (segment (start 141.603999 120.086999) (end 138.853997 122.837001) (width 0.25) (layer B.Cu) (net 37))
 (segment (start 156.610999 120.086999) (end 141.603999 120.086999) (width 0.25) (layer B.Cu) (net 37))
 (segment (start 138.853997 122.837001) (end 132.997001 122.837001) (width 0.25) (layer B.Cu) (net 37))
 (segment (start 159.968 123.444) (end 156.610999 120.086999) (width 0.25) (layer B.Cu) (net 37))
 (segment (start 202.692 91.4) (end 204.002 92.71) (width 0.3) (layer B.Cu) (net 2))
 (segment (start 202.692 78.232) (end 202.692 91.4) (width 0.3) (layer B.Cu) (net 2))
 (segment (start 201.688 98.044) (end 200.608 98.044) (width 0.3) (layer B.Cu) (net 2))
 (segment (start 204.002 95.73) (end 201.688 98.044) (width 0.3) (layer B.Cu) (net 2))
 (segment (start 204.002 92.71) (end 204.002 95.73) (width 0.3) (layer B.Cu) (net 2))
 (segment (start 117.983001 54.992001) (end 118.745 55.754) (width 0.25) (layer B.Cu) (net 4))
 (segment (start 117.557999 54.566999) (end 117.983001 54.992001) (width 0.25) (layer B.Cu) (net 4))
 (segment (start 117.557999 51.861001) (end 117.557999 54.566999) (width 0.25) (layer B.Cu) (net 4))
 (segment (start 118.745 50.674) (end 117.557999 51.861001) (width 0.25) (layer B.Cu) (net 4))
 (segment (start 141.240001 122.411999) (end 142.24 121.412) (width 0.25) (layer B.Cu) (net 4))
 (segment (start 139.336999 124.315001) (end 141.240001 122.411999) (width 0.25) (layer B.Cu) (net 4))
 (segment (start 113.744989 123.029991) (end 115.029999 124.315001) (width 0.25) (layer B.Cu) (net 4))
 (segment (start 113.744989 60.754011) (end 113.744989 123.029991) (width 0.25) (layer B.Cu) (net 4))
 (segment (start 115.029999 124.315001) (end 139.336999 124.315001) (width 0.25) (layer B.Cu) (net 4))
 (segment (start 118.745 55.754) (end 113.744989 60.754011) (width 0.25) (layer B.Cu) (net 4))
 (segment (start 148.082 51.2805) (end 148.082 53.5305) (width 0.25) (layer B.Cu) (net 5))
 (segment (start 147.4745 50.673) (end 148.082 51.2805) (width 0.25) (layer B.Cu) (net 5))
 (segment (start 137.636 50.673) (end 147.4745 50.673) (width 0.25) (layer B.Cu) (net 5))
 (segment (start 136.548999 66.030629) (end 136.548999 51.760001) (width 0.25) (layer B.Cu) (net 5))
 (segment (start 136.874001 51.434999) (end 137.636 50.673) (width 0.25) (layer B.Cu) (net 5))
 (segment (start 136.548999 51.760001) (end 136.874001 51.434999) (width 0.25) (layer B.Cu) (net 5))
 (segment (start 136.55837 66.04) (end 136.548999 66.030629) (width 0.25) (layer B.Cu) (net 5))
 (segment (start 137.636 66.04) (end 136.55837 66.04) (width 0.25) (layer B.Cu) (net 5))
 (segment (start 138.397999 64.261999) (end 137.636 63.5) (width 0.25) (layer B.Cu) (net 6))
 (segment (start 138.723001 65.742765) (end 138.723001 64.587001) (width 0.25) (layer B.Cu) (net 6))
 (segment (start 145.345746 72.36551) (end 138.723001 65.742765) (width 0.25) (layer B.Cu) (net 6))
 (segment (start 147.09449 72.36551) (end 145.345746 72.36551) (width 0.25) (layer B.Cu) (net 6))
 (segment (start 138.723001 64.587001) (end 138.397999 64.261999) (width 0.25) (layer B.Cu) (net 6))
 (segment (start 149.4195 70.0405) (end 147.09449 72.36551) (width 0.25) (layer B.Cu) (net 6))
 (segment (start 150.4315 70.0405) (end 149.4195 70.0405) (width 0.25) (layer B.Cu) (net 6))
 (segment (start 145.796 60.29537) (end 145.796 67.7905) (width 0.25) (layer B.Cu) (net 7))
 (segment (start 145.796 67.7905) (end 145.796 70.0405) (width 0.25) (layer B.Cu) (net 7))
 (segment (start 138.71363 53.213) (end 145.796 60.29537) (width 0.25) (layer B.Cu) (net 7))
 (segment (start 137.636 53.213) (end 138.71363 53.213) (width 0.25) (layer B.Cu) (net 7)))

